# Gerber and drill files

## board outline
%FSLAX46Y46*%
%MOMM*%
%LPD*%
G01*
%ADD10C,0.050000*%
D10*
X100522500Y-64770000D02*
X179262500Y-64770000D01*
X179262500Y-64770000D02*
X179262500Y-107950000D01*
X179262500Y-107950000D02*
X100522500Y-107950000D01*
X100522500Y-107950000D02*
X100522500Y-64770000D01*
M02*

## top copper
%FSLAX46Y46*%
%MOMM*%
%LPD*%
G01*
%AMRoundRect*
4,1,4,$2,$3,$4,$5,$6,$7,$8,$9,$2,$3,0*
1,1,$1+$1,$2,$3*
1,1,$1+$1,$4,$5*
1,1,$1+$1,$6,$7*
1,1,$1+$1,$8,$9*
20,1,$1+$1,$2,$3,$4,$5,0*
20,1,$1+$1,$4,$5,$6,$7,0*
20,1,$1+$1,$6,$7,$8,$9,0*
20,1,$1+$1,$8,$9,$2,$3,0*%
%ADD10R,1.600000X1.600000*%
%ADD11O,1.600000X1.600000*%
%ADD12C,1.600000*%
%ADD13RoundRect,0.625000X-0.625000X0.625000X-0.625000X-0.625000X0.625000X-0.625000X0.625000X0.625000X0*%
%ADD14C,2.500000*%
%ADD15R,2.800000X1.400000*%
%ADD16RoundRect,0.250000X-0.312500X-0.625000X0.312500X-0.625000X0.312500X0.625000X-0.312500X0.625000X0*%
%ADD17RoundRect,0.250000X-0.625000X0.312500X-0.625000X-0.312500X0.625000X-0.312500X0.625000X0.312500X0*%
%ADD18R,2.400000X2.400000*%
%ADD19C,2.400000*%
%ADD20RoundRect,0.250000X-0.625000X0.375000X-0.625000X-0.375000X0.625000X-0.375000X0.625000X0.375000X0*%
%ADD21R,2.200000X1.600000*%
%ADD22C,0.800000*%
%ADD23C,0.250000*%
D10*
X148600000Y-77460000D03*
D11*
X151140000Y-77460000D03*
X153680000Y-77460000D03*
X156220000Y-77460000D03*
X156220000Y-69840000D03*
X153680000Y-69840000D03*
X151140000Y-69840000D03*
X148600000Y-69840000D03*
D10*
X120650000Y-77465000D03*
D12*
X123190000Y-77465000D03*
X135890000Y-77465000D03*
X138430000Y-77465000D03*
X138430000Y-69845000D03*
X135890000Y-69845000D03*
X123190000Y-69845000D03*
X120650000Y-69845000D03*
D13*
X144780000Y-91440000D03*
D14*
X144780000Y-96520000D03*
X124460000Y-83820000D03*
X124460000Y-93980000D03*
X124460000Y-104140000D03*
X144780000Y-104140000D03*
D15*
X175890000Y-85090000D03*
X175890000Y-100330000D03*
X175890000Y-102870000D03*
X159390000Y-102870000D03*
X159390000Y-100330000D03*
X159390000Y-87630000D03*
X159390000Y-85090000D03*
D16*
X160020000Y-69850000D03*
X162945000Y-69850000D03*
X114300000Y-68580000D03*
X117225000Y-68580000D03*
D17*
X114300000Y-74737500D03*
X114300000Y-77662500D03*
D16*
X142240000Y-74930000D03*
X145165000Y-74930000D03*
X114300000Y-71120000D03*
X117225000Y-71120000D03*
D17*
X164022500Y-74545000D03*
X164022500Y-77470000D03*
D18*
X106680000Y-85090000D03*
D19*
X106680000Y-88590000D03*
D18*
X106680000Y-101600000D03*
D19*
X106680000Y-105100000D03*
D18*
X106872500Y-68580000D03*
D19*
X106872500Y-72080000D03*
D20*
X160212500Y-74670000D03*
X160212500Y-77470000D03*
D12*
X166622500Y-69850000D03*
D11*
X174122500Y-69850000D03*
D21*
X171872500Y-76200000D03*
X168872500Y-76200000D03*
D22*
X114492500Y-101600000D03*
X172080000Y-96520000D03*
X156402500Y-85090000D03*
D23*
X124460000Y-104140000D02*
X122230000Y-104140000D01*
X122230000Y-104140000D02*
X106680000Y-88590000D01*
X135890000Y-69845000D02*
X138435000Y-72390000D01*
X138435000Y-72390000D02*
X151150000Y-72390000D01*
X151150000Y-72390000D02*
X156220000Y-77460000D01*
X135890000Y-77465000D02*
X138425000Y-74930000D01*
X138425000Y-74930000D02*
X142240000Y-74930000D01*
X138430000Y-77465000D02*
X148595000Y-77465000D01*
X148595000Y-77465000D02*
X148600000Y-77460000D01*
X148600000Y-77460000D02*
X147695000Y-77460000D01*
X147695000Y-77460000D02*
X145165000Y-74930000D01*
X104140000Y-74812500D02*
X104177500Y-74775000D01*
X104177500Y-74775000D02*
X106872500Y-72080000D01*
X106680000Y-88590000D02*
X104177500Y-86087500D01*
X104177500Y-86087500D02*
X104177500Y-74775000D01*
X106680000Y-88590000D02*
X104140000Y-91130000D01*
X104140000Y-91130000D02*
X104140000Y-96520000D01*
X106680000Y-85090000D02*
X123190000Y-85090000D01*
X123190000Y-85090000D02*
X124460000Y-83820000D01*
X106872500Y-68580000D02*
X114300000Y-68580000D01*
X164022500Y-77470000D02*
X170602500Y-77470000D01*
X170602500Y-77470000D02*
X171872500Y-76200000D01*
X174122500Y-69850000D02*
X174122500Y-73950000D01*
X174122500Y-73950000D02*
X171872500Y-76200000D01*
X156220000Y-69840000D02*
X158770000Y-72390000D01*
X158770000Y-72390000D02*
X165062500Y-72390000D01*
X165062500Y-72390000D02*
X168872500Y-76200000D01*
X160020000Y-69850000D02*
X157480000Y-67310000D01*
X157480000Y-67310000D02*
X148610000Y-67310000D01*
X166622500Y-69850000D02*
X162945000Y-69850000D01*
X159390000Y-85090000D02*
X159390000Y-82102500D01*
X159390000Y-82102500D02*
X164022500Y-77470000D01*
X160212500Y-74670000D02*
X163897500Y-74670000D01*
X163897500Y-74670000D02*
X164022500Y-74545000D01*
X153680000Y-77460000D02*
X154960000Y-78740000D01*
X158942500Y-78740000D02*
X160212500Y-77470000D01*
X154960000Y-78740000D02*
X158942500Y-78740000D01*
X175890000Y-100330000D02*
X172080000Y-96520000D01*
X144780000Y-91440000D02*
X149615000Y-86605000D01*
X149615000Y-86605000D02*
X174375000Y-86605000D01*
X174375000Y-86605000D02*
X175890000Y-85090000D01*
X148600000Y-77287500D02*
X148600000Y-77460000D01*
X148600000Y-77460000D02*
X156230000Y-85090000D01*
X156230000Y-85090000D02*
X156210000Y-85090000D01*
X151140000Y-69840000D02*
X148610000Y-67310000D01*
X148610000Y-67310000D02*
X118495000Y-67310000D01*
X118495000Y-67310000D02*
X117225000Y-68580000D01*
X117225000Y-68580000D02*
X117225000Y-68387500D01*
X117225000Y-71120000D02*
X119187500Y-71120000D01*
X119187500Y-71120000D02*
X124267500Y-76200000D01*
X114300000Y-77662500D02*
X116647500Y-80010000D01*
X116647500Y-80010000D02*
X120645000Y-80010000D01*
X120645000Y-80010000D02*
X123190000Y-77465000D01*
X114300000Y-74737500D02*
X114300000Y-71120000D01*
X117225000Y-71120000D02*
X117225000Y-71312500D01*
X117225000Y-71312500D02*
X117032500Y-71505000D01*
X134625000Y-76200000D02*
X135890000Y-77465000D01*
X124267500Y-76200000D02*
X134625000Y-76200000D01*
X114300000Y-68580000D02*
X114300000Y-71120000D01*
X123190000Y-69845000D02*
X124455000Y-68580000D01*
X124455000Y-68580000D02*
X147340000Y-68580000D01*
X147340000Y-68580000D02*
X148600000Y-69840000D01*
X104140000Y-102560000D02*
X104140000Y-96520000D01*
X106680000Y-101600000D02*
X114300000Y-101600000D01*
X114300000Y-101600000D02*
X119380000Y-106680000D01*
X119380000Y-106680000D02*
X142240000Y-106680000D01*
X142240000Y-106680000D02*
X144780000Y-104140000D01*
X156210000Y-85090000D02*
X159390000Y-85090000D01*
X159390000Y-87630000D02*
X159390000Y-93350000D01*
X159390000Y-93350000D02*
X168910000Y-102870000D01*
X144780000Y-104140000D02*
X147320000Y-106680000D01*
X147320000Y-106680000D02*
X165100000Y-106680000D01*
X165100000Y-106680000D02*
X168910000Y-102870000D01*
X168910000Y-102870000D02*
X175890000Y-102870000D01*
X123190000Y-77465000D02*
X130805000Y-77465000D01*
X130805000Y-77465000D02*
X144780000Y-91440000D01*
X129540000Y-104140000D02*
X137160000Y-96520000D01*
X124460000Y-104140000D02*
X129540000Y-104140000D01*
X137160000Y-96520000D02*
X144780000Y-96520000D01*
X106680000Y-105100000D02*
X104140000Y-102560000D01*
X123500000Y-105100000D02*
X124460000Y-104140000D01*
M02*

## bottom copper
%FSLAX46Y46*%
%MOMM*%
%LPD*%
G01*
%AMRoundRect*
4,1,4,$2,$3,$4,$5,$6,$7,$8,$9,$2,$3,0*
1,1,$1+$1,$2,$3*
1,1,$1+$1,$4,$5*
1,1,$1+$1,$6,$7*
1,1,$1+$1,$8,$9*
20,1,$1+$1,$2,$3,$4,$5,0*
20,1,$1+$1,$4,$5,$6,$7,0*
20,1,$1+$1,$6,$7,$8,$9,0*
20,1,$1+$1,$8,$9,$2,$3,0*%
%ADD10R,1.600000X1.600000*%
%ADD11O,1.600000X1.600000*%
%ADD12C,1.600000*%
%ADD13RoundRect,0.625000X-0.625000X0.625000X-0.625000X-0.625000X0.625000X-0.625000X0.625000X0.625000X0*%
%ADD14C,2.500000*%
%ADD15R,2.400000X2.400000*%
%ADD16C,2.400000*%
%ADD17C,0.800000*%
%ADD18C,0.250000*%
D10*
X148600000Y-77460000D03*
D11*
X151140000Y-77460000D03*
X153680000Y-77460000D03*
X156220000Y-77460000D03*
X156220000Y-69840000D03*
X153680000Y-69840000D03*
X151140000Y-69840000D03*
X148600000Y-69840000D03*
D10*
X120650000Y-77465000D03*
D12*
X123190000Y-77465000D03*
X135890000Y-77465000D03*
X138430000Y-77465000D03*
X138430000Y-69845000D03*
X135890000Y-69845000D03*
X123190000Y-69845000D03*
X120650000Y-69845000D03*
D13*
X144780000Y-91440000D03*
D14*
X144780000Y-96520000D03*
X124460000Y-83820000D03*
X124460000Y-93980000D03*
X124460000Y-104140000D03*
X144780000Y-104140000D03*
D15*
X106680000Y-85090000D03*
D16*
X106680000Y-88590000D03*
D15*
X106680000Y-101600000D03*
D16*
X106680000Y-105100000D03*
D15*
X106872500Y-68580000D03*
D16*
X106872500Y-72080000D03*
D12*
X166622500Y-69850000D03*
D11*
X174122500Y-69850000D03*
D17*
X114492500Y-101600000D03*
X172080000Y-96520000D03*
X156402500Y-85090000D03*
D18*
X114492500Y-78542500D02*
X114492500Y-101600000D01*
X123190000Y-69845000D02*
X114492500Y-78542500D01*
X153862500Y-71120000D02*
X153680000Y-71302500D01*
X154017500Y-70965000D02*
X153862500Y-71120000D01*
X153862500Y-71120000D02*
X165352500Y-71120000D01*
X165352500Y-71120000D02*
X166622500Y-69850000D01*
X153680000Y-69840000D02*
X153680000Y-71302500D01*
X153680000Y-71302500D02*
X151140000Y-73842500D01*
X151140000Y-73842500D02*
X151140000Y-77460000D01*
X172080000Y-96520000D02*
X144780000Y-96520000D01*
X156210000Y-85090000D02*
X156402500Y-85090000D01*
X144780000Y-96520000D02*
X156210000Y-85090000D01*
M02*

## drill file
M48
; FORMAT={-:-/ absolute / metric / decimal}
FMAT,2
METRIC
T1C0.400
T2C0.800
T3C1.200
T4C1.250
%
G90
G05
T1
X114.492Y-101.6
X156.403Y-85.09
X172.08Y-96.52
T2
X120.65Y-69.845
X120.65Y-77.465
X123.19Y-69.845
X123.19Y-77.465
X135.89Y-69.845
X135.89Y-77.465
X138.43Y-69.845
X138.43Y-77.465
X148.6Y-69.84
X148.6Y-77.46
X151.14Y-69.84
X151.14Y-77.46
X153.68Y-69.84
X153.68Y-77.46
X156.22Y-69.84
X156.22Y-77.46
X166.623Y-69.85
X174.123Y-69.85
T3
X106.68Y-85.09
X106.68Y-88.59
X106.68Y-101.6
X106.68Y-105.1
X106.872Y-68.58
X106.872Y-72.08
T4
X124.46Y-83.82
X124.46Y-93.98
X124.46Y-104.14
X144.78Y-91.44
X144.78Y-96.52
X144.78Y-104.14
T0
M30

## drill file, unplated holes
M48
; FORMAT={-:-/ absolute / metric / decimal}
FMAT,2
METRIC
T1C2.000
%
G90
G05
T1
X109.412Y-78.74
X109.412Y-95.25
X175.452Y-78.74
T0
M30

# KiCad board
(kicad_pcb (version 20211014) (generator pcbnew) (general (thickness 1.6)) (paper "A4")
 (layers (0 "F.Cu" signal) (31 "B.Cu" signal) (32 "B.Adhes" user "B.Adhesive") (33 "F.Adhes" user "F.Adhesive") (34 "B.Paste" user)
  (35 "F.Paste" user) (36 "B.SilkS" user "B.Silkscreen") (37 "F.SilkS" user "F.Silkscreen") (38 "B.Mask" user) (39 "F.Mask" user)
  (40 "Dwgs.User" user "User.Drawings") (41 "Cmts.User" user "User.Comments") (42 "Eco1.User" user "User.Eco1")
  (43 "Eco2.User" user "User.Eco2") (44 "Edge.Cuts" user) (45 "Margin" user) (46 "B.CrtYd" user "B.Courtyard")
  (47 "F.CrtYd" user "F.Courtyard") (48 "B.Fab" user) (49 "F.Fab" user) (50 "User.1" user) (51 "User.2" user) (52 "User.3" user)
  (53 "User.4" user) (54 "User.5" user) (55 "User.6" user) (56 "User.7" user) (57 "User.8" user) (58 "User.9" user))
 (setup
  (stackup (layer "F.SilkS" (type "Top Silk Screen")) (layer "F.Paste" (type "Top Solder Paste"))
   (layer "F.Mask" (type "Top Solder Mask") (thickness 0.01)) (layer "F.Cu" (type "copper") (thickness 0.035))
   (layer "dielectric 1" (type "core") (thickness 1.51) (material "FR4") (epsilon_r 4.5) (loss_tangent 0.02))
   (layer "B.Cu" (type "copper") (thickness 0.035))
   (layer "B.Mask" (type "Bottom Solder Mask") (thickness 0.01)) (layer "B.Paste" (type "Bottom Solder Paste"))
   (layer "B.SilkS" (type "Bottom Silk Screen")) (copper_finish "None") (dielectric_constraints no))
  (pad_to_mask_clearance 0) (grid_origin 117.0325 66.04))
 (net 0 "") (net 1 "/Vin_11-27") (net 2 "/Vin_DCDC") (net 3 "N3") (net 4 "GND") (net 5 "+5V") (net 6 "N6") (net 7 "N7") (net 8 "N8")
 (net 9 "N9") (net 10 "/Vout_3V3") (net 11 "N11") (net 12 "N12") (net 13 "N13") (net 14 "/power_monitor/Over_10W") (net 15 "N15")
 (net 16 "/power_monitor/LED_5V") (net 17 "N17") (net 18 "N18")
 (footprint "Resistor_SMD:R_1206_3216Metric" (layer "F.Cu") (at 114.3 76.2 -90)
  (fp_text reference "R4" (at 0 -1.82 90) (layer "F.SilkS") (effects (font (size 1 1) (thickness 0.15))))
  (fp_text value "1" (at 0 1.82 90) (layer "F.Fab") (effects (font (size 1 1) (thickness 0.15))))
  (pad "1" smd roundrect (at -1.4625 0 270) (size 1.125 1.75) (layers "F.Cu" "F.Paste" "F.Mask") (roundrect_rratio 0.2222222222)
   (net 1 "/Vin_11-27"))
  (pad "2" smd roundrect (at 1.4625 0 270) (size 1.125 1.75) (layers "F.Cu" "F.Paste" "F.Mask") (roundrect_rratio 0.2222222222)
   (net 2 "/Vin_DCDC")))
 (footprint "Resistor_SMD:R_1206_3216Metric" (layer "F.Cu") (at 143.7025 74.93)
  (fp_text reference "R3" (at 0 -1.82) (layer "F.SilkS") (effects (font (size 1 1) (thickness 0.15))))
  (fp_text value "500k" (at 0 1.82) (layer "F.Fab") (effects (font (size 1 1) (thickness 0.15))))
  (pad "1" smd roundrect (at -1.4625 0) (size 1.125 1.75) (layers "F.Cu" "F.Paste" "F.Mask") (roundrect_rratio 0.2222222222) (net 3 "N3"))
  (pad "2" smd roundrect (at 1.4625 0) (size 1.125 1.75) (layers "F.Cu" "F.Paste" "F.Mask") (roundrect_rratio 0.2222222222) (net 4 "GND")))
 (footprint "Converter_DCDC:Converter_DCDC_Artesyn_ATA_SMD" (layer "F.Cu") (at 167.64 93.98)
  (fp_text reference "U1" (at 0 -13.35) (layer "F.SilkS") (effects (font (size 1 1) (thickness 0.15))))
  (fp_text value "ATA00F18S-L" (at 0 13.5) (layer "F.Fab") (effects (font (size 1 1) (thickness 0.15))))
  (pad "1" smd rect (at -8.25 -8.89) (size 2.8 1.4) (layers "F.Cu" "F.Paste" "F.Mask") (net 4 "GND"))
  (pad "2" smd rect (at -8.25 -6.35) (size 2.8 1.4) (layers "F.Cu" "F.Paste" "F.Mask") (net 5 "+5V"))
  (pad "7" smd rect (at -8.25 6.35) (size 2.8 1.4) (layers "F.Cu" "F.Paste" "F.Mask") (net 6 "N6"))
  (pad "8" smd rect (at -8.25 8.89) (size 2.8 1.4) (layers "F.Cu" "F.Paste" "F.Mask") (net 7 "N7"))
  (pad "9" smd rect (at 8.25 8.89) (size 2.8 1.4) (layers "F.Cu" "F.Paste" "F.Mask") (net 5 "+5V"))
  (pad "10" smd rect (at 8.25 6.35) (size 2.8 1.4) (layers "F.Cu" "F.Paste" "F.Mask") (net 4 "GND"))
  (pad "16" smd rect (at 8.25 -8.89) (size 2.8 1.4) (layers "F.Cu" "F.Paste" "F.Mask") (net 2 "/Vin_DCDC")))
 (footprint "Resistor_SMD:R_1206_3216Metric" (layer "F.Cu") (at 161.4825 69.85)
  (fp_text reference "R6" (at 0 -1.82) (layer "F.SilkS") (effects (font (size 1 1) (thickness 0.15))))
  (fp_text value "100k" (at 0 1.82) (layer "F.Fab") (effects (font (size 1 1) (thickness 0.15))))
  (pad "1" smd roundrect (at -1.4625 0) (size 1.125 1.75) (layers "F.Cu" "F.Paste" "F.Mask") (roundrect_rratio 0.2222222222) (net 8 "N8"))
  (pad "2" smd roundrect (at 1.4625 0) (size 1.125 1.75) (layers "F.Cu" "F.Paste" "F.Mask") (roundrect_rratio 0.2222222222) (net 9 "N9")))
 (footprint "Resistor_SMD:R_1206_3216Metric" (layer "F.Cu") (at 115.7625 71.12)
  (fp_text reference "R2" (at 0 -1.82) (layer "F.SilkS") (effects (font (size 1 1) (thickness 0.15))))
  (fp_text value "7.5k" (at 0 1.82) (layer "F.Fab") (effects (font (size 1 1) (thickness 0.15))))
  (pad "1" smd roundrect (at -1.4625 0) (size 1.125 1.75) (layers "F.Cu" "F.Paste" "F.Mask") (roundrect_rratio 0.2222222222)
   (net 1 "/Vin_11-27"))
  (pad "2" smd roundrect (at 1.4625 0) (size 1.125 1.75) (layers "F.Cu" "F.Paste" "F.Mask") (roundrect_rratio 0.2222222222) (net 3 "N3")))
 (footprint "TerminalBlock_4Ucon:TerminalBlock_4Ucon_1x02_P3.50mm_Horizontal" (layer "F.Cu") (at 106.68 101.6 -90)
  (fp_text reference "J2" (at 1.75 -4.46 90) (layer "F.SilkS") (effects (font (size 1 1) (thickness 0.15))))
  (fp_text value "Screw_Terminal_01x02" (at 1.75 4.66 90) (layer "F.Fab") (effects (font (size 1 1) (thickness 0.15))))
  (pad "1" thru_hole rect (at 0 0 270) (size 2.4 2.4) (drill 1.2) (layers *.Cu *.Mask) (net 5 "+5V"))
  (pad "2" thru_hole circle (at 3.5 0 270) (size 2.4 2.4) (drill 1.2) (layers *.Cu *.Mask) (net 4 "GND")))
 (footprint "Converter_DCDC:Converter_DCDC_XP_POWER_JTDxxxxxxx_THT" (layer "F.Cu") (at 144.78 91.44 -90)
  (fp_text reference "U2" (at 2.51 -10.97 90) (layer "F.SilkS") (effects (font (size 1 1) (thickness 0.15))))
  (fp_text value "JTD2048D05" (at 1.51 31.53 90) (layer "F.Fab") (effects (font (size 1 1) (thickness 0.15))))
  (pad "1" thru_hole roundrect (at 0 0 270) (size 2.5 2.5) (drill 1.25) (layers *.Cu *.Mask) (roundrect_rratio 0.25) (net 2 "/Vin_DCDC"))
  (pad "2" thru_hole circle (at 5.08 0 270) (size 2.5 2.5) (drill 1.25) (layers *.Cu *.Mask) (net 4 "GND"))
  (pad "3" thru_hole circle (at -7.62 20.32 270) (size 2.5 2.5) (drill 1.25) (layers *.Cu *.Mask) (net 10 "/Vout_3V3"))
  (pad "4" thru_hole circle (at 2.54 20.32 270) (size 2.5 2.5) (drill 1.25) (layers *.Cu *.Mask) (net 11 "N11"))
  (pad "5" thru_hole circle (at 12.7 20.32 270) (size 2.5 2.5) (drill 1.25) (layers *.Cu *.Mask) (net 4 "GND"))
  (pad "6" thru_hole circle (at 12.7 0 270) (size 2.5 2.5) (drill 1.25) (layers *.Cu *.Mask) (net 5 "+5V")))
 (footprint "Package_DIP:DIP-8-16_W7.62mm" (layer "F.Cu") (at 120.65 77.465 90)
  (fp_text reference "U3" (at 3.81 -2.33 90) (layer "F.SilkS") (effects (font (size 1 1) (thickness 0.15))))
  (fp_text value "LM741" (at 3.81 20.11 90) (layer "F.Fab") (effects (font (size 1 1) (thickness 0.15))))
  (pad "1" thru_hole rect (at 0 0 90) (size 1.6 1.6) (drill 0.8) (layers *.Cu *.Mask) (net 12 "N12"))
  (pad "2" thru_hole circle (at 0 2.54 90) (size 1.6 1.6) (drill 0.8) (layers *.Cu *.Mask) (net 2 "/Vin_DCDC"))
  (pad "3" thru_hole circle (at 0 15.24 90) (size 1.6 1.6) (drill 0.8) (layers *.Cu *.Mask) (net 3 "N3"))
  (pad "4" thru_hole circle (at 0 17.78 90) (size 1.6 1.6) (drill 0.8) (layers *.Cu *.Mask) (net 4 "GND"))
  (pad "5" thru_hole circle (at 7.62 17.78 90) (size 1.6 1.6) (drill 0.8) (layers *.Cu *.Mask) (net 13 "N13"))
  (pad "6" thru_hole circle (at 7.62 15.24 90) (size 1.6 1.6) (drill 0.8) (layers *.Cu *.Mask) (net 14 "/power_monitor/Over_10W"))
  (pad "7" thru_hole circle (at 7.62 2.54 90) (size 1.6 1.6) (drill 0.8) (layers *.Cu *.Mask) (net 5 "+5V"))
  (pad "8" thru_hole circle (at 7.62 0 90) (size 1.6 1.6) (drill 0.8) (layers *.Cu *.Mask) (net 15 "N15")))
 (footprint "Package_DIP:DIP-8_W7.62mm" (layer "F.Cu") (at 148.6 77.46 90)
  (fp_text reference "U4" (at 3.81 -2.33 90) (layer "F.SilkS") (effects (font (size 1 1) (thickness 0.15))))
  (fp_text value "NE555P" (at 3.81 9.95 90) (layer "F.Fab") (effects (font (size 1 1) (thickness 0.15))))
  (pad "1" thru_hole rect (at 0 0 90) (size 1.6 1.6) (drill 0.8) (layers *.Cu *.Mask) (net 4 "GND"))
  (pad "2" thru_hole oval (at 0 2.54 90) (size 1.6 1.6) (drill 0.8) (layers *.Cu *.Mask) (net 9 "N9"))
  (pad "3" thru_hole oval (at 0 5.08 90) (size 1.6 1.6) (drill 0.8) (layers *.Cu *.Mask) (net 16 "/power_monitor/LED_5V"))
  (pad "4" thru_hole oval (at 0 7.62 90) (size 1.6 1.6) (drill 0.8) (layers *.Cu *.Mask) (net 14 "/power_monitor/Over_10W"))
  (pad "5" thru_hole oval (at 7.62 7.62 90) (size 1.6 1.6) (drill 0.8) (layers *.Cu *.Mask) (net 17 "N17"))
  (pad "6" thru_hole oval (at 7.62 5.08 90) (size 1.6 1.6) (drill 0.8) (layers *.Cu *.Mask) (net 9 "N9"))
  (pad "7" thru_hole oval (at 7.62 2.54 90) (size 1.6 1.6) (drill 0.8) (layers *.Cu *.Mask) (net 8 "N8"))
  (pad "8" thru_hole oval (at 7.62 0 90) (size 1.6 1.6) (drill 0.8) (layers *.Cu *.Mask) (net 5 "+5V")))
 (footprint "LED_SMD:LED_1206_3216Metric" (layer "F.Cu") (at 160.2125 76.07 -90)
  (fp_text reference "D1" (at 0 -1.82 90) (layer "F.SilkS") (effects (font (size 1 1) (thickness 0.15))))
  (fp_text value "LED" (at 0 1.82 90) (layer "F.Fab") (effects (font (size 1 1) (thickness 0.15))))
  (pad "1" smd roundrect (at -1.4 0 270) (size 1.25 1.75) (layers "F.Cu" "F.Paste" "F.Mask") (roundrect_rratio 0.2) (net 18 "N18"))
  (pad "2" smd roundrect (at 1.4 0 270) (size 1.25 1.75) (layers "F.Cu" "F.Paste" "F.Mask") (roundrect_rratio 0.2)
   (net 16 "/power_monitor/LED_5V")))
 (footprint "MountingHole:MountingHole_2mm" (layer "F.Cu") (at 175.4525 78.74)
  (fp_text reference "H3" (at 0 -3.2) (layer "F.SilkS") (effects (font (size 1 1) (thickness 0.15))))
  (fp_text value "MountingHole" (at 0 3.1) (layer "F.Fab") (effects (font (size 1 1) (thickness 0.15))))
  (pad "" np_thru_hole circle (at 0 0) (size 2 2) (drill 2) (layers *.Cu *.Mask)))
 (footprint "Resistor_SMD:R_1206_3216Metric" (layer "F.Cu") (at 164.0225 76.0075 -90)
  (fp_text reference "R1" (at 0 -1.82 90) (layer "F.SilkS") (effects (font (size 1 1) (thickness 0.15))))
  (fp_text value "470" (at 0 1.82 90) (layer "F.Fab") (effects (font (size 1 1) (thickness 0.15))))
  (pad "1" smd roundrect (at -1.4625 0 270) (size 1.125 1.75) (layers "F.Cu" "F.Paste" "F.Mask") (roundrect_rratio 0.2222222222)
   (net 18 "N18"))
  (pad "2" smd roundrect (at 1.4625 0 270) (size 1.125 1.75) (layers "F.Cu" "F.Paste" "F.Mask") (roundrect_rratio 0.2222222222)
   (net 4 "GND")))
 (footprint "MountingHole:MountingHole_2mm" (layer "F.Cu") (at 109.4125 95.25)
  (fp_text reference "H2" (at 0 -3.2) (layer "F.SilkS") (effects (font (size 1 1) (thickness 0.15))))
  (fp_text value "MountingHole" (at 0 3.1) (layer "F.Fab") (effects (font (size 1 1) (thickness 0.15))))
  (pad "" np_thru_hole circle (at 0 0) (size 2 2) (drill 2) (layers *.Cu *.Mask)))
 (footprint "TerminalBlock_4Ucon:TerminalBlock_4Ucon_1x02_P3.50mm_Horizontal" (layer "F.Cu") (at 106.68 85.09 -90)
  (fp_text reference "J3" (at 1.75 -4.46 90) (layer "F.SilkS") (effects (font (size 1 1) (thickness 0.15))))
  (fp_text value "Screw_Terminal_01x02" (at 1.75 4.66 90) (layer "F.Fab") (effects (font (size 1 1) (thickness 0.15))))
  (pad "1" thru_hole rect (at 0 0 270) (size 2.4 2.4) (drill 1.2) (layers *.Cu *.Mask) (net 10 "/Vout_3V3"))
  (pad "2" thru_hole circle (at 3.5 0 270) (size 2.4 2.4) (drill 1.2) (layers *.Cu *.Mask) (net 4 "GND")))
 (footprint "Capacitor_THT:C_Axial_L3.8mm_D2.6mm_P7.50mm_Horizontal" (layer "F.Cu") (at 166.6225 69.85)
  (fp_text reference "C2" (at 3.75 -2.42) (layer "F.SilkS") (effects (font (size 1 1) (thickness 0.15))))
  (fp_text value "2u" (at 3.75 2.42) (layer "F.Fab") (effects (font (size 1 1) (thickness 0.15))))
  (pad "1" thru_hole circle (at 0 0) (size 1.6 1.6) (drill 0.8) (layers *.Cu *.Mask) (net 9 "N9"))
  (pad "2" thru_hole oval (at 7.5 0) (size 1.6 1.6) (drill 0.8) (layers *.Cu *.Mask) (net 4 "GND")))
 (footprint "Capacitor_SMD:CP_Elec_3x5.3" (layer "F.Cu") (at 170.3725 76.2)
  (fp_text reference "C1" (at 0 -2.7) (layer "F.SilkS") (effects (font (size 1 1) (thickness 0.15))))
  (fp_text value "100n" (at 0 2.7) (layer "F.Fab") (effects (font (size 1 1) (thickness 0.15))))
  (pad "1" smd rect (at -1.5 0) (size 2.2 1.6) (layers "F.Cu" "F.Paste" "F.Mask") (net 17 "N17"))
  (pad "2" smd rect (at 1.5 0) (size 2.2 1.6) (layers "F.Cu" "F.Paste" "F.Mask") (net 4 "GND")))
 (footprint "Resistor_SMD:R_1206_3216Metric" (layer "F.Cu") (at 115.7625 68.58)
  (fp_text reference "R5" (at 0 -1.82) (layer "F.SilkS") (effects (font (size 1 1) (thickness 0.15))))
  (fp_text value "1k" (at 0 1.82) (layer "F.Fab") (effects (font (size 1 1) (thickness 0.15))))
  (pad "1" smd roundrect (at -1.4625 0) (size 1.125 1.75) (layers "F.Cu" "F.Paste" "F.Mask") (roundrect_rratio 0.2222222222)
   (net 1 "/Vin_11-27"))
  (pad "2" smd roundrect (at 1.4625 0) (size 1.125 1.75) (layers "F.Cu" "F.Paste" "F.Mask") (roundrect_rratio 0.2222222222) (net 8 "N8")))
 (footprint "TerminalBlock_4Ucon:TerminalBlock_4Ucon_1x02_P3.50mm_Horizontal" (layer "F.Cu") (at 106.8725 68.58 -90)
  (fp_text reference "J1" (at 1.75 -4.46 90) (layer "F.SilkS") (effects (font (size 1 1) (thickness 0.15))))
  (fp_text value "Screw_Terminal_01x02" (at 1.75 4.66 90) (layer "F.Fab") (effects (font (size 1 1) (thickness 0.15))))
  (pad "1" thru_hole rect (at 0 0 270) (size 2.4 2.4) (drill 1.2) (layers *.Cu *.Mask) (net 1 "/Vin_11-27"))
  (pad "2" thru_hole circle (at 3.5 0 270) (size 2.4 2.4) (drill 1.2) (layers *.Cu *.Mask) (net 4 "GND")))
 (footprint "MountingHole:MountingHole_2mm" (layer "F.Cu") (at 109.4125 78.74)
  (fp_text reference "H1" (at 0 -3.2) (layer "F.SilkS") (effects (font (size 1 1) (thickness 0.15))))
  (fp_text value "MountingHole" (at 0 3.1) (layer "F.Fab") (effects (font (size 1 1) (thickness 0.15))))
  (pad "" np_thru_hole circle (at 0 0) (size 2 2) (drill 2) (layers *.Cu *.Mask)))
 (gr_rect (start 100.5225 64.77) (end 179.2625 107.95) (layer "Edge.Cuts") (width 0.05) (fill none))
 (segment (start 156.22 69.84) (end 158.77 72.39) (width 0.25) (layer "F.Cu") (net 17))
 (segment (start 158.77 72.39) (end 165.0625 72.39) (width 0.25) (layer "F.Cu") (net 17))
 (segment (start 165.0625 72.39) (end 168.8725 76.2) (width 0.25) (layer "F.Cu") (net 17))
 (segment (start 174.1225 69.85) (end 174.1225 73.95) (width 0.25) (layer "F.Cu") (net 4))
 (segment (start 106.68 88.59) (end 104.14 91.13) (width 0.25) (layer "F.Cu") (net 4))
 (segment (start 175.89 100.33) (end 172.08 96.52) (width 0.25) (layer "F.Cu") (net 4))
 (segment (start 170.6025 77.47) (end 171.8725 76.2) (width 0.25) (layer "F.Cu") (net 4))
 (segment (start 124.46 104.14) (end 129.54 104.14) (width 0.25) (layer "F.Cu") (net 4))
 (segment (start 123.5 105.1) (end 124.46 104.14) (width 0.25) (layer "F.Cu") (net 4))
 (segment (start 106.68 88.59) (end 104.1775 86.0875) (width 0.25) (layer "F.Cu") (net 4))
 (segment (start 124.46 104.14) (end 122.23 104.14) (width 0.25) (layer "F.Cu") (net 4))
 (segment (start 156.23 85.09) (end 156.21 85.09) (width 0.25) (layer "F.Cu") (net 4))
 (segment (start 159.39 85.09) (end 159.39 82.1025) (width 0.25) (layer "F.Cu") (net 4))
 (segment (start 164.0225 77.47) (end 170.6025 77.47) (width 0.25) (layer "F.Cu") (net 4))
 (segment (start 159.39 82.1025) (end 164.0225 77.47) (width 0.25) (layer "F.Cu") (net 4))
 (segment (start 104.1775 86.0875) (end 104.1775 74.775) (width 0.25) (layer "F.Cu") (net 4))
 (segment (start 104.1775 74.775) (end 106.8725 72.08) (width 0.25) (layer "F.Cu") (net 4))
 (segment (start 104.14 74.8125) (end 104.1775 74.775) (width 0.25) (layer "F.Cu") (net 4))
 (segment (start 148.6 77.46) (end 156.23 85.09) (width 0.25) (layer "F.Cu") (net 4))
 (segment (start 137.16 96.52) (end 144.78 96.52) (width 0.25) (layer "F.Cu") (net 4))
 (segment (start 148.6 77.46) (end 147.695 77.46) (width 0.25) (layer "F.Cu") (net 4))
 (segment (start 122.23 104.14) (end 106.68 88.59) (width 0.25) (layer "F.Cu") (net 4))
 (segment (start 156.21 85.09) (end 159.39 85.09) (width 0.25) (layer "F.Cu") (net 4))
 (segment (start 106.68 105.1) (end 104.14 102.56) (width 0.25) (layer "F.Cu") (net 4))
 (segment (start 104.14 102.56) (end 104.14 96.52) (width 0.25) (layer "F.Cu") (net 4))
 (segment (start 129.54 104.14) (end 137.16 96.52) (width 0.25) (layer "F.Cu") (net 4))
 (segment (start 147.695 77.46) (end 145.165 74.93) (width 0.25) (layer "F.Cu") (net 4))
 (segment (start 148.595 77.465) (end 148.6 77.46) (width 0.25) (layer "F.Cu") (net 4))
 (segment (start 148.6 77.2875) (end 148.6 77.46) (width 0.25) (layer "F.Cu") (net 4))
 (segment (start 104.14 91.13) (end 104.14 96.52) (width 0.25) (layer "F.Cu") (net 4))
 (segment (start 174.1225 73.95) (end 171.8725 76.2) (width 0.25) (layer "F.Cu") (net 4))
 (segment (start 138.43 77.465) (end 148.595 77.465) (width 0.25) (layer "F.Cu") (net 4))
 (via (at 156.4025 85.09) (size 0.8) (drill 0.4) (layers "F.Cu" "B.Cu") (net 4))
 (via (at 172.08 96.52) (size 0.8) (drill 0.4) (layers "F.Cu" "B.Cu") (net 4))
 (segment (start 156.21 85.09) (end 156.4025 85.09) (width 0.25) (layer "B.Cu") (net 4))
 (segment (start 144.78 96.52) (end 156.21 85.09) (width 0.25) (layer "B.Cu") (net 4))
 (segment (start 172.08 96.52) (end 144.78 96.52) (width 0.25) (layer "B.Cu") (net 4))
 (segment (start 166.6225 69.85) (end 162.945 69.85) (width 0.25) (layer "F.Cu") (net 9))
 (segment (start 153.8625 71.12) (end 165.3525 71.12) (width 0.25) (layer "B.Cu") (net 9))
 (segment (start 165.3525 71.12) (end 166.6225 69.85) (width 0.25) (layer "B.Cu") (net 9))
 (segment (start 151.14 73.8425) (end 151.14 77.46) (width 0.25) (layer "B.Cu") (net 9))
 (segment (start 153.8625 71.12) (end 153.68 71.3025) (width 0.25) (layer "B.Cu") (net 9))
 (segment (start 153.68 71.3025) (end 151.14 73.8425) (width 0.25) (layer "B.Cu") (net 9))
 (segment (start 154.0175 70.965) (end 153.8625 71.12) (width 0.25) (layer "B.Cu") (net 9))
 (segment (start 153.68 69.84) (end 153.68 71.3025) (width 0.25) (layer "B.Cu") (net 9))
 (segment (start 160.2125 74.67) (end 163.8975 74.67) (width 0.25) (layer "F.Cu") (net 18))
 (segment (start 163.8975 74.67) (end 164.0225 74.545) (width 0.25) (layer "F.Cu") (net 18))
 (segment (start 158.9425 78.74) (end 160.2125 77.47) (width 0.25) (layer "F.Cu") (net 16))
 (segment (start 154.96 78.74) (end 158.9425 78.74) (width 0.25) (layer "F.Cu") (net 16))
 (segment (start 153.68 77.46) (end 154.96 78.74) (width 0.25) (layer "F.Cu") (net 16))
 (segment (start 138.425 74.93) (end 142.24 74.93) (width 0.25) (layer "F.Cu") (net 3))
 (segment (start 124.2675 76.2) (end 134.625 76.2) (width 0.25) (layer "F.Cu") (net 3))
 (segment (start 117.225 71.12) (end 119.1875 71.12) (width 0.25) (layer "F.Cu") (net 3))
 (segment (start 135.89 77.465) (end 138.425 74.93) (width 0.25) (layer "F.Cu") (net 3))
 (segment (start 119.1875 71.12) (end 124.2675 76.2) (width 0.25) (layer "F.Cu") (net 3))
 (segment (start 117.225 71.12) (end 117.225 71.3125) (width 0.25) (layer "F.Cu") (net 3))
 (segment (start 117.225 71.3125) (end 117.0325 71.505) (width 0.25) (layer "F.Cu") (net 3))
 (segment (start 134.625 76.2) (end 135.89 77.465) (width 0.25) (layer "F.Cu") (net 3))
 (segment (start 114.3 77.6625) (end 116.6475 80.01) (width 0.25) (layer "F.Cu") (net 2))
 (segment (start 116.6475 80.01) (end 120.645 80.01) (width 0.25) (layer "F.Cu") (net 2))
 (segment (start 123.19 77.465) (end 130.805 77.465) (width 0.25) (layer "F.Cu") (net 2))
 (segment (start 174.375 86.605) (end 175.89 85.09) (width 0.25) (layer "F.Cu") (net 2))
 (segment (start 130.805 77.465) (end 144.78 91.44) (width 0.25) (layer "F.Cu") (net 2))
 (segment (start 149.615 86.605) (end 174.375 86.605) (width 0.25) (layer "F.Cu") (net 2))
 (segment (start 144.78 91.44) (end 149.615 86.605) (width 0.25) (layer "F.Cu") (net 2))
 (segment (start 120.645 80.01) (end 123.19 77.465) (width 0.25) (layer "F.Cu") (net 2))
 (segment (start 117.225 68.58) (end 117.225 68.3875) (width 0.25) (layer "F.Cu") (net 8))
 (segment (start 148.61 67.31) (end 118.495 67.31) (width 0.25) (layer "F.Cu") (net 8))
 (segment (start 160.02 69.85) (end 157.48 67.31) (width 0.25) (layer "F.Cu") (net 8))
 (segment (start 157.48 67.31) (end 148.61 67.31) (width 0.25) (layer "F.Cu") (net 8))
 (segment (start 151.14 69.84) (end 148.61 67.31) (width 0.25) (layer "F.Cu") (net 8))
 (segment (start 118.495 67.31) (end 117.225 68.58) (width 0.25) (layer "F.Cu") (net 8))
 (segment (start 142.24 106.68) (end 144.78 104.14) (width 0.25) (layer "F.Cu") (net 5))
 (segment (start 124.455 68.58) (end 147.34 68.58) (width 0.25) (layer "F.Cu") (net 5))
 (segment (start 159.39 87.63) (end 159.39 93.35) (width 0.25) (layer "F.Cu") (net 5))
 (segment (start 159.39 93.35) (end 168.91 102.87) (width 0.25) (layer "F.Cu") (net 5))
 (segment (start 114.3 101.6) (end 119.38 106.68) (width 0.25) (layer "F.Cu") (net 5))
 (segment (start 147.34 68.58) (end 148.6 69.84) (width 0.25) (layer "F.Cu") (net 5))
 (segment (start 144.78 104.14) (end 147.32 106.68) (width 0.25) (layer "F.Cu") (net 5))
 (segment (start 123.19 69.845) (end 124.455 68.58) (width 0.25) (layer "F.Cu") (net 5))
 (segment (start 165.1 106.68) (end 168.91 102.87) (width 0.25) (layer "F.Cu") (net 5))
 (segment (start 119.38 106.68) (end 142.24 106.68) (width 0.25) (layer "F.Cu") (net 5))
 (segment (start 147.32 106.68) (end 165.1 106.68) (width 0.25) (layer "F.Cu") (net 5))
 (segment (start 168.91 102.87) (end 175.89 102.87) (width 0.25) (layer "F.Cu") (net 5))
 (segment (start 106.68 101.6) (end 114.3 101.6) (width 0.25) (layer "F.Cu") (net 5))
 (via (at 114.4925 101.6) (size 0.8) (drill 0.4) (layers "F.Cu" "B.Cu") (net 5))
 (segment (start 123.19 69.845) (end 114.4925 78.5425) (width 0.25) (layer "B.Cu") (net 5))
 (segment (start 114.4925 78.5425) (end 114.4925 101.6) (width 0.25) (layer "B.Cu") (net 5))
 (segment (start 106.68 85.09) (end 123.19 85.09) (width 0.25) (layer "F.Cu") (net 10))
 (segment (start 123.19 85.09) (end 124.46 83.82) (width 0.25) (layer "F.Cu") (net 10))
 (segment (start 138.435 72.39) (end 151.15 72.39) (width 0.25) (layer "F.Cu") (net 14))
 (segment (start 151.15 72.39) (end 156.22 77.46) (width 0.25) (layer "F.Cu") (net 14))
 (segment (start 135.89 69.845) (end 138.435 72.39) (width 0.25) (layer "F.Cu") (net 14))
 (segment (start 106.8725 68.58) (end 114.3 68.58) (width 0.25) (layer "F.Cu") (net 1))
 (segment (start 114.3 68.58) (end 114.3 71.12) (width 0.25) (layer "F.Cu") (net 1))
 (segment (start 114.3 74.7375) (end 114.3 71.12) (width 0.25) (layer "F.Cu") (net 1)))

